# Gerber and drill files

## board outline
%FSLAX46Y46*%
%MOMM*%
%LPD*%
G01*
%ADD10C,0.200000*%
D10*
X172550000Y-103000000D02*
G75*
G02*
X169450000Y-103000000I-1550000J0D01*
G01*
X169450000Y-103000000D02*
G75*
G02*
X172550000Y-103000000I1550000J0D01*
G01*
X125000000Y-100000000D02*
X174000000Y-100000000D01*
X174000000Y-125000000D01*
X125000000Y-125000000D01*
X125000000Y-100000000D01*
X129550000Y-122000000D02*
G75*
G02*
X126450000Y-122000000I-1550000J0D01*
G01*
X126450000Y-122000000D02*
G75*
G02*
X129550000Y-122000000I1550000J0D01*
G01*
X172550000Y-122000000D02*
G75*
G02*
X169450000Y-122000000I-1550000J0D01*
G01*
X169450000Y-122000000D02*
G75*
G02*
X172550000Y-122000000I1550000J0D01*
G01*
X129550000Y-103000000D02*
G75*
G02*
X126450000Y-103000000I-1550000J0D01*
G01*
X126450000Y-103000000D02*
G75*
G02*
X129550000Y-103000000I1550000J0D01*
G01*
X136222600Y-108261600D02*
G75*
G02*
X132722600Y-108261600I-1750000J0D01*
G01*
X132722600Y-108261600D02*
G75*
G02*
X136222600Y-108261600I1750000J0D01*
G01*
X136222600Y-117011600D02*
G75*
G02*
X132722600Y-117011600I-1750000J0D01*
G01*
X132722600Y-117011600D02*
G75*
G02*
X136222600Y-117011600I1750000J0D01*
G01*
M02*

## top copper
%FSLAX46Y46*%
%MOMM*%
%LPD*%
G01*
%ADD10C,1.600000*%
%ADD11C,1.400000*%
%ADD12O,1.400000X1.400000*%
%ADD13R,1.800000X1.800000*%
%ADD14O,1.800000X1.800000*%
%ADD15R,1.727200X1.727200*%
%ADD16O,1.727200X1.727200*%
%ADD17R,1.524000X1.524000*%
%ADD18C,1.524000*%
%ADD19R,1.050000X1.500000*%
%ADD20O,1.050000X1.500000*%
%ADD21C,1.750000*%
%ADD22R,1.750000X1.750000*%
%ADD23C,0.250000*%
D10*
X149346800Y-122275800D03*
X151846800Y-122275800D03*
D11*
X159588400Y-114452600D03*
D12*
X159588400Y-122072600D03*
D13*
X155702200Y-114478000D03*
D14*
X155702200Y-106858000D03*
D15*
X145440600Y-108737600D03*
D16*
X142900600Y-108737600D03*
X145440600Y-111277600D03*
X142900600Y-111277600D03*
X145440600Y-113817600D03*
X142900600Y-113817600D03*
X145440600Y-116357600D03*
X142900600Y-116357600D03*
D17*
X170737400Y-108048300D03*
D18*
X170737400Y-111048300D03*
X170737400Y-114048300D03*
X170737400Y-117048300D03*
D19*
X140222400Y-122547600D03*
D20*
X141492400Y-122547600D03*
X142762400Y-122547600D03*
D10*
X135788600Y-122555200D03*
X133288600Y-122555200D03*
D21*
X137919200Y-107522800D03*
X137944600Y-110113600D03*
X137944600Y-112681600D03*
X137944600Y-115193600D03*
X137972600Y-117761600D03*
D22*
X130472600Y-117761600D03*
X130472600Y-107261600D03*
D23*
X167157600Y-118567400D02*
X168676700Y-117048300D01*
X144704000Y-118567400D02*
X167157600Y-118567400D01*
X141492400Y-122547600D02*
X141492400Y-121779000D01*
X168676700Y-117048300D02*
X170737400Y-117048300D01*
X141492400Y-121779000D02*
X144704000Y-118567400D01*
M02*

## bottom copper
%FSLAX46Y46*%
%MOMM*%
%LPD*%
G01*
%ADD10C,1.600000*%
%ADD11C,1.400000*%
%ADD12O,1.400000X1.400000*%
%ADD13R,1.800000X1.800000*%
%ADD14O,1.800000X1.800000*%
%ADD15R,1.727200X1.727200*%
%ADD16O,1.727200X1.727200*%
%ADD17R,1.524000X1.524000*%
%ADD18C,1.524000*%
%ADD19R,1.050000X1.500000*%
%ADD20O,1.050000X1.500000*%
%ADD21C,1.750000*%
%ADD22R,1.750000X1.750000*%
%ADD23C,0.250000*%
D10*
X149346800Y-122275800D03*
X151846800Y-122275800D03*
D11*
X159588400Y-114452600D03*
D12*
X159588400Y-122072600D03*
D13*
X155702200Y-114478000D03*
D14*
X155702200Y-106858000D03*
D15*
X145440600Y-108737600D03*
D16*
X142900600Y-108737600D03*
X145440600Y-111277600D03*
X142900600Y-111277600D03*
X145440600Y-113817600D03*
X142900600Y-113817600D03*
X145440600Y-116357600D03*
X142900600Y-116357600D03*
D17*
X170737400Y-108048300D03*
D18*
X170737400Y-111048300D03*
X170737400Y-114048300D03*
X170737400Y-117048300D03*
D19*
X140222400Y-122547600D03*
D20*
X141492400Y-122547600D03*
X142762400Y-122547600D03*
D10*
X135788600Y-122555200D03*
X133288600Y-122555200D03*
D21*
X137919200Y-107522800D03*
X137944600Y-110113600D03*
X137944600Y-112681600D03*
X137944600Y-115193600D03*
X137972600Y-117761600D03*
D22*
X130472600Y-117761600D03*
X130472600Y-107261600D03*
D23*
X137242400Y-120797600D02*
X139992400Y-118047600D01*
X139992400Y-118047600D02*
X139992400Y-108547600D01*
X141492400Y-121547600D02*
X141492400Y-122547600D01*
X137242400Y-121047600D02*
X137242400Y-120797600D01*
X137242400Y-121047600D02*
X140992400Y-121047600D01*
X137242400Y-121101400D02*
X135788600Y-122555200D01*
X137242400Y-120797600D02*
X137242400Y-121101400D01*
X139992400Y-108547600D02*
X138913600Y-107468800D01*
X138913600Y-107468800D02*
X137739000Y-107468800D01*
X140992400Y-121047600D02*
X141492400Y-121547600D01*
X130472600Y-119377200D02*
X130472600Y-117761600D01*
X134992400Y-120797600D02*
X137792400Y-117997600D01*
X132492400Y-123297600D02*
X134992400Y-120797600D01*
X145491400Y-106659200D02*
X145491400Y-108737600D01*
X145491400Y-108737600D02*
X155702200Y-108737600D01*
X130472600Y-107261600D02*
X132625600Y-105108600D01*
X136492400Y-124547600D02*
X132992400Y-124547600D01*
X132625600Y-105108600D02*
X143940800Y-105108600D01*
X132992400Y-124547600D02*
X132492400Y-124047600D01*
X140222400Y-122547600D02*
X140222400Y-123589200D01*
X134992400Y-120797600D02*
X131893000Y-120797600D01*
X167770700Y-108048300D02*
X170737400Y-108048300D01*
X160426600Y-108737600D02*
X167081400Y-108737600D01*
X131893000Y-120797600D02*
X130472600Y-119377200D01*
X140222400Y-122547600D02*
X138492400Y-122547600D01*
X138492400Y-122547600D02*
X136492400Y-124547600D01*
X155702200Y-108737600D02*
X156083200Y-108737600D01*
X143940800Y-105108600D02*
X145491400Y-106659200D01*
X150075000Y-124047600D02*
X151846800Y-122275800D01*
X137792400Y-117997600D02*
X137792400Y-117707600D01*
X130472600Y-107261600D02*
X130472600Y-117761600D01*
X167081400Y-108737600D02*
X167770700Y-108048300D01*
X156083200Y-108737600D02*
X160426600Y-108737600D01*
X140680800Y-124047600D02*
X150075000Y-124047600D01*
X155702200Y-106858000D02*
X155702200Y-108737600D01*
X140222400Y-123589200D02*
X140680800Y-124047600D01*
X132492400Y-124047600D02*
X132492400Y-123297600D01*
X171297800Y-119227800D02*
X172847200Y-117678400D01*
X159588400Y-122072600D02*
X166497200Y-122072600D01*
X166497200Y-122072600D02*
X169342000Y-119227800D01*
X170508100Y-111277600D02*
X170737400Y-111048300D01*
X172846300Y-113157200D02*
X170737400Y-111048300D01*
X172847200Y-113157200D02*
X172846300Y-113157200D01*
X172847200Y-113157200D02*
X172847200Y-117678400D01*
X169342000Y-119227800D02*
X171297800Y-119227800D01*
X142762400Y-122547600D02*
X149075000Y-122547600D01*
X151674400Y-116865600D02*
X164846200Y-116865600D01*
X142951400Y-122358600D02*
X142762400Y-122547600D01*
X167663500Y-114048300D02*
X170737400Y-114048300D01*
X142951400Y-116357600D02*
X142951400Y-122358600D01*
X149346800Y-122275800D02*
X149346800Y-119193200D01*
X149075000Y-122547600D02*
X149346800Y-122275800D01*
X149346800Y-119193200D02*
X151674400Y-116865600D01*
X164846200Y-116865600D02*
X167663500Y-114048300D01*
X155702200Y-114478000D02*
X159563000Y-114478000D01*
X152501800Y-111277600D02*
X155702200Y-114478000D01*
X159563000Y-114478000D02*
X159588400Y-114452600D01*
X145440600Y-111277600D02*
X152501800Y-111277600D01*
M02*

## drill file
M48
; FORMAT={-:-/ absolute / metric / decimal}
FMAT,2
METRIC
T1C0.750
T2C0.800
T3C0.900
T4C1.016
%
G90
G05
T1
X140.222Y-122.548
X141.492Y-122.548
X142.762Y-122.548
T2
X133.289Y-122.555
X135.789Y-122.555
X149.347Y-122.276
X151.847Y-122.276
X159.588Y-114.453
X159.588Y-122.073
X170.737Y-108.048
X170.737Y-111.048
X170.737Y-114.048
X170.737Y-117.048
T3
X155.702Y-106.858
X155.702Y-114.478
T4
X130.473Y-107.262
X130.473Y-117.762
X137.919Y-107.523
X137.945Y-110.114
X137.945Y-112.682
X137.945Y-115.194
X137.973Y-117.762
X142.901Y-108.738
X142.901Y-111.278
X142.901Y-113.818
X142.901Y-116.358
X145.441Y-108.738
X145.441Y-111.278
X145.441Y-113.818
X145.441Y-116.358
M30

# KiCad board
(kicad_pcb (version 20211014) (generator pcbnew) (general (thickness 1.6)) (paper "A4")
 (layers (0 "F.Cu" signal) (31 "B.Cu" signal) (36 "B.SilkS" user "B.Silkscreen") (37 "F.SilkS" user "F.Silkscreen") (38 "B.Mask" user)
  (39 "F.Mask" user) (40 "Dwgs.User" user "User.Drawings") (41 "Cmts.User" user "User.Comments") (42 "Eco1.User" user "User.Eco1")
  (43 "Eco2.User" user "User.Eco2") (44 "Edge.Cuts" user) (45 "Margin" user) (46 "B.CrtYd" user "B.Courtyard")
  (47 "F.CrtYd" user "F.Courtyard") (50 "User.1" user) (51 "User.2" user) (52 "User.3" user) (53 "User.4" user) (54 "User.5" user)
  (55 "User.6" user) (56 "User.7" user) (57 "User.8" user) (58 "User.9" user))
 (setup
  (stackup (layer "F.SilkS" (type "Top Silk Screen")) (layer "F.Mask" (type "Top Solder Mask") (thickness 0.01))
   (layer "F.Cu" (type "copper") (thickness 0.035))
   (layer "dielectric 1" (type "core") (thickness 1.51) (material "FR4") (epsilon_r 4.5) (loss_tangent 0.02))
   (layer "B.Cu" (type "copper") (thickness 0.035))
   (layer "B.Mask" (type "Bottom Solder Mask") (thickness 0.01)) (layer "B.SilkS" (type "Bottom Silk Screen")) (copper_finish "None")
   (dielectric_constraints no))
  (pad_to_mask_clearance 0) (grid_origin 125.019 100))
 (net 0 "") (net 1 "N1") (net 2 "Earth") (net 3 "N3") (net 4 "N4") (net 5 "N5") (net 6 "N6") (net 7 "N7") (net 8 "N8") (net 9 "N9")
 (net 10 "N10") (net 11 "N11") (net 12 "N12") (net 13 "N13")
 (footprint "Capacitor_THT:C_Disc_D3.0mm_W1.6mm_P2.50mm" (layer "F.Cu") (at 149.3468 122.2758)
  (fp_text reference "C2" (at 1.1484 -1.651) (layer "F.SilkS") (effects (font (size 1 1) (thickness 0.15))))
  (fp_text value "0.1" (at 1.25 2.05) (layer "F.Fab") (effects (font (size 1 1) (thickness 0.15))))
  (pad "1" thru_hole circle (at 0 0) (size 1.6 1.6) (drill 0.8) (layers *.Cu *.Mask) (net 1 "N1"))
  (pad "2" thru_hole circle (at 2.5 0) (size 1.6 1.6) (drill 0.8) (layers *.Cu *.Mask) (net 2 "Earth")))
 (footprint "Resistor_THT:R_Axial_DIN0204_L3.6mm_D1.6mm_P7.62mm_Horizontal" (layer "F.Cu") (at 159.5884 114.4526 -90)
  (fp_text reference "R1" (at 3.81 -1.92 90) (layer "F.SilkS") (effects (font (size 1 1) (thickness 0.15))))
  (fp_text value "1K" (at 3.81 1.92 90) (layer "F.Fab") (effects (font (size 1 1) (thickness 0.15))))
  (pad "1" thru_hole circle (at 0 0 270) (size 1.4 1.4) (drill 0.8) (layers *.Cu *.Mask) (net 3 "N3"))
  (pad "2" thru_hole oval (at 7.62 0 270) (size 1.4 1.4) (drill 0.8) (layers *.Cu *.Mask) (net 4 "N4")))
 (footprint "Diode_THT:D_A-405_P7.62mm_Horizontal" (layer "F.Cu") (at 155.7022 114.478 90)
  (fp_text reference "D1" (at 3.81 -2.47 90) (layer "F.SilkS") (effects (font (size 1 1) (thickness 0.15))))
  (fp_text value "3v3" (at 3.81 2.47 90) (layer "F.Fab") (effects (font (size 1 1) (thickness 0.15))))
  (pad "1" thru_hole rect (at 0 0 90) (size 1.8 1.8) (drill 0.9) (layers *.Cu *.Mask) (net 3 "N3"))
  (pad "2" thru_hole oval (at 7.62 0 90) (size 1.8 1.8) (drill 0.9) (layers *.Cu *.Mask) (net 2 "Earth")))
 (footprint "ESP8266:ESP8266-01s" (layer "F.Cu") (at 142.9006 108.7376)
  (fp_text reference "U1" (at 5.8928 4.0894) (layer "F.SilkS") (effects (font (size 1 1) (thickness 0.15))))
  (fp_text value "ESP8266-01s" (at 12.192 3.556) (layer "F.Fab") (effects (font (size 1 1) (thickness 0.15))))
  (pad "1" thru_hole rect (at 2.54 0) (size 1.7272 1.7272) (drill 1.016) (layers *.Cu *.Mask) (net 2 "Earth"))
  (pad "2" thru_hole oval (at 0 0) (size 1.7272 1.7272) (drill 1.016) (layers *.Cu *.Mask) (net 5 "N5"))
  (pad "3" thru_hole oval (at 2.54 2.54) (size 1.7272 1.7272) (drill 1.016) (layers *.Cu *.Mask) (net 3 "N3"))
  (pad "4" thru_hole oval (at 0 2.54) (size 1.7272 1.7272) (drill 1.016) (layers *.Cu *.Mask) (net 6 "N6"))
  (pad "5" thru_hole oval (at 2.54 5.08) (size 1.7272 1.7272) (drill 1.016) (layers *.Cu *.Mask) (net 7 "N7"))
  (pad "6" thru_hole oval (at 0 5.08) (size 1.7272 1.7272) (drill 1.016) (layers *.Cu *.Mask) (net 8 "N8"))
  (pad "7" thru_hole oval (at 2.54 7.62) (size 1.7272 1.7272) (drill 1.016) (layers *.Cu *.Mask) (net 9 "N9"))
  (pad "8" thru_hole oval (at 0 7.62) (size 1.7272 1.7272) (drill 1.016) (layers *.Cu *.Mask) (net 1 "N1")))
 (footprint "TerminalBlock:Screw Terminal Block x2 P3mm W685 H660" (layer "F.Cu") (at 170.7374 108.0483 -90)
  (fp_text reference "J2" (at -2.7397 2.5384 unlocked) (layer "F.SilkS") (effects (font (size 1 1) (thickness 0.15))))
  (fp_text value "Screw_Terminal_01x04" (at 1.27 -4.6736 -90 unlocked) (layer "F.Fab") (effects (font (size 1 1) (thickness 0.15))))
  (pad "1" thru_hole rect (at 0 0 270) (size 1.524 1.524) (drill 0.8) (layers *.Cu *.Mask) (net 2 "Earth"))
  (pad "2" thru_hole circle (at 3 0 270) (size 1.524 1.524) (drill 0.8) (layers *.Cu *.Mask) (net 4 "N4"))
  (pad "3" thru_hole circle (at 6 0 270) (size 1.524 1.524) (drill 0.8) (layers *.Cu *.Mask) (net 1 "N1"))
  (pad "4" thru_hole circle (at 9 0 270) (size 1.524 1.524) (drill 0.8) (layers *.Cu *.Mask) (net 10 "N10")))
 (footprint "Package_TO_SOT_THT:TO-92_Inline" (layer "F.Cu") (at 140.2224 122.5476)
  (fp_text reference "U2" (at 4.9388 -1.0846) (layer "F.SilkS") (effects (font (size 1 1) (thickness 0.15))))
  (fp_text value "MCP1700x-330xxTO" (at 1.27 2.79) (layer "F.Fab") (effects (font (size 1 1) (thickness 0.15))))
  (pad "1" thru_hole rect (at 0 0) (size 1.05 1.5) (drill 0.75) (layers *.Cu *.Mask) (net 2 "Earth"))
  (pad "2" thru_hole oval (at 1.27 0) (size 1.05 1.5) (drill 0.75) (layers *.Cu *.Mask) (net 10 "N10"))
  (pad "3" thru_hole oval (at 2.54 0) (size 1.05 1.5) (drill 0.75) (layers *.Cu *.Mask) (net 1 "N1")))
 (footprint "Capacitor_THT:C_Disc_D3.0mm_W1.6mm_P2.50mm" (layer "F.Cu") (at 135.7886 122.5552 180)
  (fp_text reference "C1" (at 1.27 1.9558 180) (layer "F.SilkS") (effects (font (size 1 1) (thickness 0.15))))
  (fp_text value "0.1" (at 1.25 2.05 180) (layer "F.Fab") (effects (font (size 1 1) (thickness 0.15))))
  (pad "1" thru_hole circle (at 0 0 180) (size 1.6 1.6) (drill 0.8) (layers *.Cu *.Mask) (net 10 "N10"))
  (pad "2" thru_hole circle (at 2.5 0 180) (size 1.6 1.6) (drill 0.8) (layers *.Cu *.Mask) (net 2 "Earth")))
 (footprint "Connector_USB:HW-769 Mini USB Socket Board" (layer "F.Cu") (at 139.7226 119.5116)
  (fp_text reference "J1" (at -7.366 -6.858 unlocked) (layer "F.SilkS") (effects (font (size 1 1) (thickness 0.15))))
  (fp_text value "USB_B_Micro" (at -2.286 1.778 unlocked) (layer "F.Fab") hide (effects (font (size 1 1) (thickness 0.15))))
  (fp_circle (center -5.25 -11.25) (end -3.5 -11.25) (layer "Edge.Cuts") (width 0.2) (fill none))
  (fp_circle (center -5.25 -2.5) (end -3.5 -2.5) (layer "Edge.Cuts") (width 0.2) (fill none))
  (pad "1" thru_hole circle (at -1.8034 -11.9888) (size 1.75 1.75) (drill 1.016) (layers *.Cu *.Mask) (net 10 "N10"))
  (pad "2" thru_hole circle (at -1.778 -9.398) (size 1.75 1.75) (drill 1.016) (layers *.Cu *.Mask) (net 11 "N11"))
  (pad "3" thru_hole circle (at -1.778 -6.83) (size 1.75 1.75) (drill 1.016) (layers *.Cu *.Mask) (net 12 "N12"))
  (pad "4" thru_hole circle (at -1.778 -4.318) (size 1.75 1.75) (drill 1.016) (layers *.Cu *.Mask) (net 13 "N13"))
  (pad "5" thru_hole circle (at -1.75 -1.75) (size 1.75 1.75) (drill 1.016) (layers *.Cu *.Mask) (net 2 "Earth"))
  (pad "6" thru_hole rect (at -9.25 -1.75) (size 1.75 1.75) (drill 1.016) (layers *.Cu *.Mask) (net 2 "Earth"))
  (pad "7" thru_hole rect (at -9.25 -12.25) (size 1.75 1.75) (drill 1.016) (layers *.Cu *.Mask) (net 2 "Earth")))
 (gr_circle (center 171 103) (end 172.55 103) (layer "Edge.Cuts") (width 0.2) (fill none))
 (gr_rect (start 125 100) (end 174 125) (layer "Edge.Cuts") (width 0.2) (fill none))
 (gr_circle (center 128 122) (end 129.55 122) (layer "Edge.Cuts") (width 0.2) (fill none))
 (gr_circle (center 171 122) (end 172.55 122) (layer "Edge.Cuts") (width 0.2) (fill none))
 (gr_circle (center 128 103) (end 129.55 103) (layer "Edge.Cuts") (width 0.2) (fill none))
 (segment (start 167.1576 118.5674) (end 168.6767 117.0483) (width 0.25) (layer "F.Cu") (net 10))
 (segment (start 144.704 118.5674) (end 167.1576 118.5674) (width 0.25) (layer "F.Cu") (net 10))
 (segment (start 141.4924 122.5476) (end 141.4924 121.779) (width 0.25) (layer "F.Cu") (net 10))
 (segment (start 168.6767 117.0483) (end 170.7374 117.0483) (width 0.25) (layer "F.Cu") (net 10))
 (segment (start 141.4924 121.779) (end 144.704 118.5674) (width 0.25) (layer "F.Cu") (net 10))
 (segment (start 137.2424 120.7976) (end 139.9924 118.0476) (width 0.25) (layer "B.Cu") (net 10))
 (segment (start 139.9924 118.0476) (end 139.9924 108.5476) (width 0.25) (layer "B.Cu") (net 10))
 (segment (start 141.4924 121.5476) (end 141.4924 122.5476) (width 0.25) (layer "B.Cu") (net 10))
 (segment (start 137.2424 121.0476) (end 137.2424 120.7976) (width 0.25) (layer "B.Cu") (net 10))
 (segment (start 137.2424 121.0476) (end 140.9924 121.0476) (width 0.25) (layer "B.Cu") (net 10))
 (segment (start 137.2424 121.1014) (end 135.7886 122.5552) (width 0.25) (layer "B.Cu") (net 10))
 (segment (start 137.2424 120.7976) (end 137.2424 121.1014) (width 0.25) (layer "B.Cu") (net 10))
 (segment (start 139.9924 108.5476) (end 138.9136 107.4688) (width 0.25) (layer "B.Cu") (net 10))
 (segment (start 138.9136 107.4688) (end 137.739 107.4688) (width 0.25) (layer "B.Cu") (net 10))
 (segment (start 140.9924 121.0476) (end 141.4924 121.5476) (width 0.25) (layer "B.Cu") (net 10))
 (segment (start 130.4726 119.3772) (end 130.4726 117.7616) (width 0.25) (layer "B.Cu") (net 2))
 (segment (start 134.9924 120.7976) (end 137.7924 117.9976) (width 0.25) (layer "B.Cu") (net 2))
 (segment (start 132.4924 123.2976) (end 134.9924 120.7976) (width 0.25) (layer "B.Cu") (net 2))
 (segment (start 145.4914 106.6592) (end 145.4914 108.7376) (width 0.25) (layer "B.Cu") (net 2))
 (segment (start 145.4914 108.7376) (end 155.7022 108.7376) (width 0.25) (layer "B.Cu") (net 2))
 (segment (start 130.4726 107.2616) (end 132.6256 105.1086) (width 0.25) (layer "B.Cu") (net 2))
 (segment (start 136.4924 124.5476) (end 132.9924 124.5476) (width 0.25) (layer "B.Cu") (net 2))
 (segment (start 132.6256 105.1086) (end 143.9408 105.1086) (width 0.25) (layer "B.Cu") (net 2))
 (segment (start 132.9924 124.5476) (end 132.4924 124.0476) (width 0.25) (layer "B.Cu") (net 2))
 (segment (start 140.2224 122.5476) (end 140.2224 123.5892) (width 0.25) (layer "B.Cu") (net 2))
 (segment (start 134.9924 120.7976) (end 131.893 120.7976) (width 0.25) (layer "B.Cu") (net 2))
 (segment (start 167.7707 108.0483) (end 170.7374 108.0483) (width 0.25) (layer "B.Cu") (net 2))
 (segment (start 160.4266 108.7376) (end 167.0814 108.7376) (width 0.25) (layer "B.Cu") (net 2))
 (segment (start 131.893 120.7976) (end 130.4726 119.3772) (width 0.25) (layer "B.Cu") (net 2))
 (segment (start 140.2224 122.5476) (end 138.4924 122.5476) (width 0.25) (layer "B.Cu") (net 2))
 (segment (start 138.4924 122.5476) (end 136.4924 124.5476) (width 0.25) (layer "B.Cu") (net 2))
 (segment (start 155.7022 108.7376) (end 156.0832 108.7376) (width 0.25) (layer "B.Cu") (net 2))
 (segment (start 143.9408 105.1086) (end 145.4914 106.6592) (width 0.25) (layer "B.Cu") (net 2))
 (segment (start 150.075 124.0476) (end 151.8468 122.2758) (width 0.25) (layer "B.Cu") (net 2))
 (segment (start 137.7924 117.9976) (end 137.7924 117.7076) (width 0.25) (layer "B.Cu") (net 2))
 (segment (start 130.4726 107.2616) (end 130.4726 117.7616) (width 0.25) (layer "B.Cu") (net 2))
 (segment (start 167.0814 108.7376) (end 167.7707 108.0483) (width 0.25) (layer "B.Cu") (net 2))
 (segment (start 156.0832 108.7376) (end 160.4266 108.7376) (width 0.25) (layer "B.Cu") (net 2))
 (segment (start 140.6808 124.0476) (end 150.075 124.0476) (width 0.25) (layer "B.Cu") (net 2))
 (segment (start 155.7022 106.858) (end 155.7022 108.7376) (width 0.25) (layer "B.Cu") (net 2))
 (segment (start 140.2224 123.5892) (end 140.6808 124.0476) (width 0.25) (layer "B.Cu") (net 2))
 (segment (start 132.4924 124.0476) (end 132.4924 123.2976) (width 0.25) (layer "B.Cu") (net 2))
 (segment (start 171.2978 119.2278) (end 172.8472 117.6784) (width 0.25) (layer "B.Cu") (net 4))
 (segment (start 159.5884 122.0726) (end 166.4972 122.0726) (width 0.25) (layer "B.Cu") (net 4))
 (segment (start 166.4972 122.0726) (end 169.342 119.2278) (width 0.25) (layer "B.Cu") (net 4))
 (segment (start 170.5081 111.2776) (end 170.7374 111.0483) (width 0.25) (layer "B.Cu") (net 4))
 (segment (start 172.8463 113.1572) (end 170.7374 111.0483) (width 0.25) (layer "B.Cu") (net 4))
 (segment (start 172.8472 113.1572) (end 172.8463 113.1572) (width 0.25) (layer "B.Cu") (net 4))
 (segment (start 172.8472 113.1572) (end 172.8472 117.6784) (width 0.25) (layer "B.Cu") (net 4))
 (segment (start 169.342 119.2278) (end 171.2978 119.2278) (width 0.25) (layer "B.Cu") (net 4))
 (segment (start 142.7624 122.5476) (end 149.075 122.5476) (width 0.25) (layer "B.Cu") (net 1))
 (segment (start 151.6744 116.8656) (end 164.8462 116.8656) (width 0.25) (layer "B.Cu") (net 1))
 (segment (start 142.9514 122.3586) (end 142.7624 122.5476) (width 0.25) (layer "B.Cu") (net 1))
 (segment (start 167.6635 114.0483) (end 170.7374 114.0483) (width 0.25) (layer "B.Cu") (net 1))
 (segment (start 142.9514 116.3576) (end 142.9514 122.3586) (width 0.25) (layer "B.Cu") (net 1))
 (segment (start 149.3468 122.2758) (end 149.3468 119.1932) (width 0.25) (layer "B.Cu") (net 1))
 (segment (start 149.075 122.5476) (end 149.3468 122.2758) (width 0.25) (layer "B.Cu") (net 1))
 (segment (start 149.3468 119.1932) (end 151.6744 116.8656) (width 0.25) (layer "B.Cu") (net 1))
 (segment (start 164.8462 116.8656) (end 167.6635 114.0483) (width 0.25) (layer "B.Cu") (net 1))
 (segment (start 155.7022 114.478) (end 159.563 114.478) (width 0.25) (layer "B.Cu") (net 3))
 (segment (start 152.5018 111.2776) (end 155.7022 114.478) (width 0.25) (layer "B.Cu") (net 3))
 (segment (start 159.563 114.478) (end 159.5884 114.4526) (width 0.25) (layer "B.Cu") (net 3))
 (segment (start 145.4406 111.2776) (end 152.5018 111.2776) (width 0.25) (layer "B.Cu") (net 3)))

